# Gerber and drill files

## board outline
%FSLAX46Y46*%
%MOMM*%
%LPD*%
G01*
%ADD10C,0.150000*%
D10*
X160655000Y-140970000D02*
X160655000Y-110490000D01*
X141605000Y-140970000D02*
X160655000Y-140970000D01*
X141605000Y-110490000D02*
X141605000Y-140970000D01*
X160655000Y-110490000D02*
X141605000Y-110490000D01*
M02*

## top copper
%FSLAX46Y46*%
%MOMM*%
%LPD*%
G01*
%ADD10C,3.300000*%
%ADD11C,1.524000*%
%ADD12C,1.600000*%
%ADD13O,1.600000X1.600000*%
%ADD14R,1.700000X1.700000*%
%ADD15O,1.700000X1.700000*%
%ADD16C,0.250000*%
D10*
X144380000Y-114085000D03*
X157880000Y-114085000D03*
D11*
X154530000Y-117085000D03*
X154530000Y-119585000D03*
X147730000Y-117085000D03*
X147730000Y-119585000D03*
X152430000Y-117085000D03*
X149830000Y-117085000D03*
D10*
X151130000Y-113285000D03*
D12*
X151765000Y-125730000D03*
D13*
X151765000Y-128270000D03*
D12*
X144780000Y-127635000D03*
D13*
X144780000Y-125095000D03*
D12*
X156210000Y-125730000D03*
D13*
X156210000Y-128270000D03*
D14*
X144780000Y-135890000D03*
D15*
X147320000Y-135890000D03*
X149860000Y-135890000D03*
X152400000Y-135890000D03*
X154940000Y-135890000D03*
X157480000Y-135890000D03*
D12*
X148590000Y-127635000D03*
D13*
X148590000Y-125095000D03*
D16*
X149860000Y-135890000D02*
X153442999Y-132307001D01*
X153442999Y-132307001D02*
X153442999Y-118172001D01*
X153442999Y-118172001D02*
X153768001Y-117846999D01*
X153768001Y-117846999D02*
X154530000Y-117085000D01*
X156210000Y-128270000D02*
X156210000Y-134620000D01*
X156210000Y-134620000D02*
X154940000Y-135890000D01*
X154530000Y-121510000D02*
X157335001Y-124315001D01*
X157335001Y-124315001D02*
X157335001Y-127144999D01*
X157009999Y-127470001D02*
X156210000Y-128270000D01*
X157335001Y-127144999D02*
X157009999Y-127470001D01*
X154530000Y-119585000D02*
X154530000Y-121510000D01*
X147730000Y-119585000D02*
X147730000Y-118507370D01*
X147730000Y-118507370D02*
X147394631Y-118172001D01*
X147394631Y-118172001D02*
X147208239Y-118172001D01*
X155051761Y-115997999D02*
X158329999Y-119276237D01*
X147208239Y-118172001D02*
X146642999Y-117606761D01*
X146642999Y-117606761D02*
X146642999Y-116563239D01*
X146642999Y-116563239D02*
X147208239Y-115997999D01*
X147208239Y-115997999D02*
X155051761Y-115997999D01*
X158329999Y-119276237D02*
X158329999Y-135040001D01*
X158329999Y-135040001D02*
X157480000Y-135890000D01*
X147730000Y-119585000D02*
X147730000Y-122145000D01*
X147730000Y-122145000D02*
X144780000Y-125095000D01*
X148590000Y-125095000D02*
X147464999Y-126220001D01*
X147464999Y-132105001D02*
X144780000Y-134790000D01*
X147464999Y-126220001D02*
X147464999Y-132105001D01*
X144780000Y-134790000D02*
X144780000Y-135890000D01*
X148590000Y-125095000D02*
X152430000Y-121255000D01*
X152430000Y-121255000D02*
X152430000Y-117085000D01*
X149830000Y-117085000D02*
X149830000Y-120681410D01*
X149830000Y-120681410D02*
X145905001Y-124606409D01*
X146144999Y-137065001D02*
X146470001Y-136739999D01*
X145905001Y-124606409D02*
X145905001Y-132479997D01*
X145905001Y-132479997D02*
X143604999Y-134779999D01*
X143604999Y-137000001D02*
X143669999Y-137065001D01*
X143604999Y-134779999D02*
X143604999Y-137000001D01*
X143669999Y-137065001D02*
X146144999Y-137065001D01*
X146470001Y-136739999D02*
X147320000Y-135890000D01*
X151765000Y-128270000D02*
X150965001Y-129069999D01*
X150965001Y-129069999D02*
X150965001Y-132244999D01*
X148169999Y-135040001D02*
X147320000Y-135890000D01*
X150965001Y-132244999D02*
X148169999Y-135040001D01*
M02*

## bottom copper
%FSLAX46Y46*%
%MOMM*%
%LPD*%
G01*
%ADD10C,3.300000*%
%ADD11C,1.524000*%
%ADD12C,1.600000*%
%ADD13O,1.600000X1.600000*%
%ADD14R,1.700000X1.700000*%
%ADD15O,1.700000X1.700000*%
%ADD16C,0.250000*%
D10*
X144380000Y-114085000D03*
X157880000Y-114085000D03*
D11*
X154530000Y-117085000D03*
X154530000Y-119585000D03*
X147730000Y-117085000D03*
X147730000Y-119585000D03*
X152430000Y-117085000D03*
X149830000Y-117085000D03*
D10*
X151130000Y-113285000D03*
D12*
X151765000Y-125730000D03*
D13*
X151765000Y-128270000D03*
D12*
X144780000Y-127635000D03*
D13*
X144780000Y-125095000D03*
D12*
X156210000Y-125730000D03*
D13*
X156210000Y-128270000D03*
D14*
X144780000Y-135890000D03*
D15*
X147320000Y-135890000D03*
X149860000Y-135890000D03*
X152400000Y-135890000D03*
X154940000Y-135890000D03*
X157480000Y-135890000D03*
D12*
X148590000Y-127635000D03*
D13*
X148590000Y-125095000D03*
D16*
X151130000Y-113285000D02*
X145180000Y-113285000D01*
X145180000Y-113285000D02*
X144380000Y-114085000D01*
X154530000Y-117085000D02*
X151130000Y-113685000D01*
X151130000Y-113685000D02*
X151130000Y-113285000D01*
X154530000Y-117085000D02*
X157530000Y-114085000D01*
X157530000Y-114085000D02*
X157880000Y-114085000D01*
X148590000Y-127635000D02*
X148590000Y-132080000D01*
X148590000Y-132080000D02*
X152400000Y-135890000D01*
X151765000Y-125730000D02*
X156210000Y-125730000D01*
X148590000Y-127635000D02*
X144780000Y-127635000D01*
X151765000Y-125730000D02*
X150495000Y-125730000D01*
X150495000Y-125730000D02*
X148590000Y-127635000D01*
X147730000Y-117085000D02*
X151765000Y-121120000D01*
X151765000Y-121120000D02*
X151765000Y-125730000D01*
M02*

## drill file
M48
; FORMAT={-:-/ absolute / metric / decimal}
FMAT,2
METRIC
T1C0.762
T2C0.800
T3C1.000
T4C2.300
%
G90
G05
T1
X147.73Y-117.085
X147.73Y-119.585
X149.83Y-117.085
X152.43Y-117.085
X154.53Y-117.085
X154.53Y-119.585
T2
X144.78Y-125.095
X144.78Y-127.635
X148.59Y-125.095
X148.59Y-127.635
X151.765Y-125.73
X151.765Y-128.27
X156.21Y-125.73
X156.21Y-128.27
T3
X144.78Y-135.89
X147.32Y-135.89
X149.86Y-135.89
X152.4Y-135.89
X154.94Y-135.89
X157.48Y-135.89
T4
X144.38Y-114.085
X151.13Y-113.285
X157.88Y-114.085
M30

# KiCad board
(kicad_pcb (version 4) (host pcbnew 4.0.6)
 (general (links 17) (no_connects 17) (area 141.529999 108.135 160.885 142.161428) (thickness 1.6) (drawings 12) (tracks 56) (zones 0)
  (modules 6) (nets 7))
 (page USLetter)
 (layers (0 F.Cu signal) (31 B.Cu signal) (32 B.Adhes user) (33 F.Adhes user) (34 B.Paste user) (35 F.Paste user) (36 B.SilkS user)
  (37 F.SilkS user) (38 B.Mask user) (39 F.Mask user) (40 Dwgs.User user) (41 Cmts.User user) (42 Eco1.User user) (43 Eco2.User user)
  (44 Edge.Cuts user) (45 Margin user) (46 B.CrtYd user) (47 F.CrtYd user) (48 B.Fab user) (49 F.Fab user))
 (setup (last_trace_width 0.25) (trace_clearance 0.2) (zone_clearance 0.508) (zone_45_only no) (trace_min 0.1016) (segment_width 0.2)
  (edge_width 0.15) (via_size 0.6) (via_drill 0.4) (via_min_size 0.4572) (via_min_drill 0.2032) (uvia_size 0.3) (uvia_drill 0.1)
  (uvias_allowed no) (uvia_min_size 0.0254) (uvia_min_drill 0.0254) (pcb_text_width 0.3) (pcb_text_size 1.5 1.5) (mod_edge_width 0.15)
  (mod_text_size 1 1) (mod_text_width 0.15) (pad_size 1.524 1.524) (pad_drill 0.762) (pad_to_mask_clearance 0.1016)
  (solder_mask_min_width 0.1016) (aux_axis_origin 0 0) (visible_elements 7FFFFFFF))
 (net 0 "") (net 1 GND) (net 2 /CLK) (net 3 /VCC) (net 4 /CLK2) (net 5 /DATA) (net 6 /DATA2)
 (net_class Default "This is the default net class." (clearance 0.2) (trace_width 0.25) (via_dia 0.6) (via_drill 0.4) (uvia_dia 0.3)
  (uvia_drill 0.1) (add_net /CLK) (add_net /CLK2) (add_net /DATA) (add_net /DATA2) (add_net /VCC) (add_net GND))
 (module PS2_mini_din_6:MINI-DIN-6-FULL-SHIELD (layer F.Cu) (at 151.13 108.585)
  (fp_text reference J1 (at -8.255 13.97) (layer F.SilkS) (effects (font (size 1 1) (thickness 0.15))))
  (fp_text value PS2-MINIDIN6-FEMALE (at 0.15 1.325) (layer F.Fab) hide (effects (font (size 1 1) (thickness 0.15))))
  (pad 7 thru_hole circle (at -6.75 5.5) (size 3.3 3.3) (drill 2.3) (layers *.Cu *.Mask) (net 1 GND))
  (pad 7 thru_hole circle (at 6.75 5.5) (size 3.3 3.3) (drill 2.3) (layers *.Cu *.Mask) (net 1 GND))
  (pad 3 thru_hole circle (at 3.4 8.5) (size 1.524 1.524) (drill 0.762) (layers *.Cu *.Mask) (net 1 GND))
  (pad 5 thru_hole circle (at 3.4 11) (size 1.524 1.524) (drill 0.762) (layers *.Cu *.Mask) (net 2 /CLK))
  (pad 4 thru_hole circle (at -3.4 8.5) (size 1.524 1.524) (drill 0.762) (layers *.Cu *.Mask) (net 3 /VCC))
  (pad 6 thru_hole circle (at -3.4 11) (size 1.524 1.524) (drill 0.762) (layers *.Cu *.Mask) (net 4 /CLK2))
  (pad 1 thru_hole circle (at 1.3 8.5) (size 1.524 1.524) (drill 0.762) (layers *.Cu *.Mask) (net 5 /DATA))
  (pad 2 thru_hole circle (at -1.3 8.5) (size 1.524 1.524) (drill 0.762) (layers *.Cu *.Mask) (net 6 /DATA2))
  (pad 7 thru_hole circle (at 0 4.7) (size 3.3 3.3) (drill 2.3) (layers *.Cu *.Mask) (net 1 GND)))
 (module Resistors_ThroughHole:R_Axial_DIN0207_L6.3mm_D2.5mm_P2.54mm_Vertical (layer F.Cu) (at 151.765 125.73 270)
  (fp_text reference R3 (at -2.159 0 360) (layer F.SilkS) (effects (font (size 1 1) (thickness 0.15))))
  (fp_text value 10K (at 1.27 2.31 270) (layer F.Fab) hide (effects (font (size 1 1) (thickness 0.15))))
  (pad 1 thru_hole circle (at 0 0 270) (size 1.6 1.6) (drill 0.8) (layers *.Cu *.Mask) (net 3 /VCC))
  (pad 2 thru_hole oval (at 2.54 0 270) (size 1.6 1.6) (drill 0.8) (layers *.Cu *.Mask) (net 6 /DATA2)))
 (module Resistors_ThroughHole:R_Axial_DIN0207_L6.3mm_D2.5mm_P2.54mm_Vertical (layer F.Cu) (at 144.78 127.635 90)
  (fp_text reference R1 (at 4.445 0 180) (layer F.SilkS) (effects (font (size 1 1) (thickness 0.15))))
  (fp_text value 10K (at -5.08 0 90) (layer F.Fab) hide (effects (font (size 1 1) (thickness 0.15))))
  (pad 1 thru_hole circle (at 0 0 90) (size 1.6 1.6) (drill 0.8) (layers *.Cu *.Mask) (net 3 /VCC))
  (pad 2 thru_hole oval (at 2.54 0 90) (size 1.6 1.6) (drill 0.8) (layers *.Cu *.Mask) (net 4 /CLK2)))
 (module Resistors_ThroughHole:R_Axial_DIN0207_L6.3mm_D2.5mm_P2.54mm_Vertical (layer F.Cu) (at 156.21 125.73 270)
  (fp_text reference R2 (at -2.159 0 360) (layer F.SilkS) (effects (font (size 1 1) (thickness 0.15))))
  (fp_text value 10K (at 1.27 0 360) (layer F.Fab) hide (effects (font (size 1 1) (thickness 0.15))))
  (pad 1 thru_hole circle (at 0 0 270) (size 1.6 1.6) (drill 0.8) (layers *.Cu *.Mask) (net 3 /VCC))
  (pad 2 thru_hole oval (at 2.54 0 270) (size 1.6 1.6) (drill 0.8) (layers *.Cu *.Mask) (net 2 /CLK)))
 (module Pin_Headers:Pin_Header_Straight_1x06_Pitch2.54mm (layer F.Cu) (at 144.78 135.89 90)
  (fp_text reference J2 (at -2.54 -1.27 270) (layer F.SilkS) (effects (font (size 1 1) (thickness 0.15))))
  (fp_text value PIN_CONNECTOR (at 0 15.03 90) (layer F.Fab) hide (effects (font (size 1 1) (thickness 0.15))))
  (pad 1 thru_hole rect (at 0 0 90) (size 1.7 1.7) (drill 1) (layers *.Cu *.Mask) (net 5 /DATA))
  (pad 2 thru_hole oval (at 0 2.54 90) (size 1.7 1.7) (drill 1) (layers *.Cu *.Mask) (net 6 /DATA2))
  (pad 3 thru_hole oval (at 0 5.08 90) (size 1.7 1.7) (drill 1) (layers *.Cu *.Mask) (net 1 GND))
  (pad 4 thru_hole oval (at 0 7.62 90) (size 1.7 1.7) (drill 1) (layers *.Cu *.Mask) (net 3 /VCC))
  (pad 5 thru_hole oval (at 0 10.16 90) (size 1.7 1.7) (drill 1) (layers *.Cu *.Mask) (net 2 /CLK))
  (pad 6 thru_hole oval (at 0 12.7 90) (size 1.7 1.7) (drill 1) (layers *.Cu *.Mask) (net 4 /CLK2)))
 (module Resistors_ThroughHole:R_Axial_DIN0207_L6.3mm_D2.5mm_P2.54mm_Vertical (layer F.Cu) (at 148.59 127.635 90)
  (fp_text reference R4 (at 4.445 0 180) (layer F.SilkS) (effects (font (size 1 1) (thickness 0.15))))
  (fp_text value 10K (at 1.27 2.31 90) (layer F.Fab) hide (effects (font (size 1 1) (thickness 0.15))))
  (pad 1 thru_hole circle (at 0 0 90) (size 1.6 1.6) (drill 0.8) (layers *.Cu *.Mask) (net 3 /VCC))
  (pad 2 thru_hole oval (at 2.54 0 90) (size 1.6 1.6) (drill 0.8) (layers *.Cu *.Mask) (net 5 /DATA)))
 (gr_line (start 160.655 140.97) (end 160.655 110.49) (layer Edge.Cuts) (width 0.15))
 (gr_line (start 141.605 140.97) (end 160.655 140.97) (layer Edge.Cuts) (width 0.15))
 (gr_line (start 141.605 110.49) (end 141.605 140.97) (layer Edge.Cuts) (width 0.15))
 (gr_line (start 160.655 110.49) (end 141.605 110.49) (layer Edge.Cuts) (width 0.15))
 (segment (start 151.13 113.285) (end 145.18 113.285) (width 0.25) (layer B.Cu) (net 1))
 (segment (start 145.18 113.285) (end 144.38 114.085) (width 0.25) (layer B.Cu) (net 1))
 (segment (start 154.53 117.085) (end 151.13 113.685) (width 0.25) (layer B.Cu) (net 1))
 (segment (start 151.13 113.685) (end 151.13 113.285) (width 0.25) (layer B.Cu) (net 1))
 (segment (start 154.53 117.085) (end 157.53 114.085) (width 0.25) (layer B.Cu) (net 1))
 (segment (start 157.53 114.085) (end 157.88 114.085) (width 0.25) (layer B.Cu) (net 1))
 (segment (start 149.86 135.89) (end 153.442999 132.307001) (width 0.25) (layer F.Cu) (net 1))
 (segment (start 153.442999 132.307001) (end 153.442999 118.172001) (width 0.25) (layer F.Cu) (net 1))
 (segment (start 153.442999 118.172001) (end 153.768001 117.846999) (width 0.25) (layer F.Cu) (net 1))
 (segment (start 153.768001 117.846999) (end 154.53 117.085) (width 0.25) (layer F.Cu) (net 1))
 (segment (start 156.21 128.27) (end 156.21 134.62) (width 0.25) (layer F.Cu) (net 2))
 (segment (start 156.21 134.62) (end 154.94 135.89) (width 0.25) (layer F.Cu) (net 2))
 (segment (start 154.53 121.51) (end 157.335001 124.315001) (width 0.25) (layer F.Cu) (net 2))
 (segment (start 157.335001 124.315001) (end 157.335001 127.144999) (width 0.25) (layer F.Cu) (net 2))
 (segment (start 157.009999 127.470001) (end 156.21 128.27) (width 0.25) (layer F.Cu) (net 2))
 (segment (start 157.335001 127.144999) (end 157.009999 127.470001) (width 0.25) (layer F.Cu) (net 2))
 (segment (start 154.53 119.585) (end 154.53 121.51) (width 0.25) (layer F.Cu) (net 2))
 (segment (start 148.59 127.635) (end 148.59 132.08) (width 0.25) (layer B.Cu) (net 3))
 (segment (start 148.59 132.08) (end 152.4 135.89) (width 0.25) (layer B.Cu) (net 3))
 (segment (start 151.765 125.73) (end 156.21 125.73) (width 0.25) (layer B.Cu) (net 3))
 (segment (start 148.59 127.635) (end 144.78 127.635) (width 0.25) (layer B.Cu) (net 3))
 (segment (start 151.765 125.73) (end 150.495 125.73) (width 0.25) (layer B.Cu) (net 3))
 (segment (start 150.495 125.73) (end 148.59 127.635) (width 0.25) (layer B.Cu) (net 3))
 (segment (start 147.73 117.085) (end 151.765 121.12) (width 0.25) (layer B.Cu) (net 3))
 (segment (start 151.765 121.12) (end 151.765 125.73) (width 0.25) (layer B.Cu) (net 3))
 (segment (start 147.73 119.585) (end 147.73 118.50737) (width 0.25) (layer F.Cu) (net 4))
 (segment (start 147.73 118.50737) (end 147.394631 118.172001) (width 0.25) (layer F.Cu) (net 4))
 (segment (start 147.394631 118.172001) (end 147.208239 118.172001) (width 0.25) (layer F.Cu) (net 4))
 (segment (start 155.051761 115.997999) (end 158.329999 119.276237) (width 0.25) (layer F.Cu) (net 4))
 (segment (start 147.208239 118.172001) (end 146.642999 117.606761) (width 0.25) (layer F.Cu) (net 4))
 (segment (start 146.642999 117.606761) (end 146.642999 116.563239) (width 0.25) (layer F.Cu) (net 4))
 (segment (start 146.642999 116.563239) (end 147.208239 115.997999) (width 0.25) (layer F.Cu) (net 4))
 (segment (start 147.208239 115.997999) (end 155.051761 115.997999) (width 0.25) (layer F.Cu) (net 4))
 (segment (start 158.329999 119.276237) (end 158.329999 135.040001) (width 0.25) (layer F.Cu) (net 4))
 (segment (start 158.329999 135.040001) (end 157.48 135.89) (width 0.25) (layer F.Cu) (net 4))
 (segment (start 147.73 119.585) (end 147.73 122.145) (width 0.25) (layer F.Cu) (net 4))
 (segment (start 147.73 122.145) (end 144.78 125.095) (width 0.25) (layer F.Cu) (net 4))
 (segment (start 148.59 125.095) (end 147.464999 126.220001) (width 0.25) (layer F.Cu) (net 5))
 (segment (start 147.464999 132.105001) (end 144.78 134.79) (width 0.25) (layer F.Cu) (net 5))
 (segment (start 147.464999 126.220001) (end 147.464999 132.105001) (width 0.25) (layer F.Cu) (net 5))
 (segment (start 144.78 134.79) (end 144.78 135.89) (width 0.25) (layer F.Cu) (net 5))
 (segment (start 148.59 125.095) (end 152.43 121.255) (width 0.25) (layer F.Cu) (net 5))
 (segment (start 152.43 121.255) (end 152.43 117.085) (width 0.25) (layer F.Cu) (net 5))
 (segment (start 149.83 117.085) (end 149.83 120.68141) (width 0.25) (layer F.Cu) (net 6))
 (segment (start 149.83 120.68141) (end 145.905001 124.606409) (width 0.25) (layer F.Cu) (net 6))
 (segment (start 146.144999 137.065001) (end 146.470001 136.739999) (width 0.25) (layer F.Cu) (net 6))
 (segment (start 145.905001 124.606409) (end 145.905001 132.479997) (width 0.25) (layer F.Cu) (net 6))
 (segment (start 145.905001 132.479997) (end 143.604999 134.779999) (width 0.25) (layer F.Cu) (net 6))
 (segment (start 143.604999 137.000001) (end 143.669999 137.065001) (width 0.25) (layer F.Cu) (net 6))
 (segment (start 143.604999 134.779999) (end 143.604999 137.000001) (width 0.25) (layer F.Cu) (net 6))
 (segment (start 143.669999 137.065001) (end 146.144999 137.065001) (width 0.25) (layer F.Cu) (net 6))
 (segment (start 146.470001 136.739999) (end 147.32 135.89) (width 0.25) (layer F.Cu) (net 6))
 (segment (start 151.765 128.27) (end 150.965001 129.069999) (width 0.25) (layer F.Cu) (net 6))
 (segment (start 150.965001 129.069999) (end 150.965001 132.244999) (width 0.25) (layer F.Cu) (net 6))
 (segment (start 148.169999 135.040001) (end 147.32 135.89) (width 0.25) (layer F.Cu) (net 6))
 (segment (start 150.965001 132.244999) (end 148.169999 135.040001) (width 0.25) (layer F.Cu) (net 6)))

